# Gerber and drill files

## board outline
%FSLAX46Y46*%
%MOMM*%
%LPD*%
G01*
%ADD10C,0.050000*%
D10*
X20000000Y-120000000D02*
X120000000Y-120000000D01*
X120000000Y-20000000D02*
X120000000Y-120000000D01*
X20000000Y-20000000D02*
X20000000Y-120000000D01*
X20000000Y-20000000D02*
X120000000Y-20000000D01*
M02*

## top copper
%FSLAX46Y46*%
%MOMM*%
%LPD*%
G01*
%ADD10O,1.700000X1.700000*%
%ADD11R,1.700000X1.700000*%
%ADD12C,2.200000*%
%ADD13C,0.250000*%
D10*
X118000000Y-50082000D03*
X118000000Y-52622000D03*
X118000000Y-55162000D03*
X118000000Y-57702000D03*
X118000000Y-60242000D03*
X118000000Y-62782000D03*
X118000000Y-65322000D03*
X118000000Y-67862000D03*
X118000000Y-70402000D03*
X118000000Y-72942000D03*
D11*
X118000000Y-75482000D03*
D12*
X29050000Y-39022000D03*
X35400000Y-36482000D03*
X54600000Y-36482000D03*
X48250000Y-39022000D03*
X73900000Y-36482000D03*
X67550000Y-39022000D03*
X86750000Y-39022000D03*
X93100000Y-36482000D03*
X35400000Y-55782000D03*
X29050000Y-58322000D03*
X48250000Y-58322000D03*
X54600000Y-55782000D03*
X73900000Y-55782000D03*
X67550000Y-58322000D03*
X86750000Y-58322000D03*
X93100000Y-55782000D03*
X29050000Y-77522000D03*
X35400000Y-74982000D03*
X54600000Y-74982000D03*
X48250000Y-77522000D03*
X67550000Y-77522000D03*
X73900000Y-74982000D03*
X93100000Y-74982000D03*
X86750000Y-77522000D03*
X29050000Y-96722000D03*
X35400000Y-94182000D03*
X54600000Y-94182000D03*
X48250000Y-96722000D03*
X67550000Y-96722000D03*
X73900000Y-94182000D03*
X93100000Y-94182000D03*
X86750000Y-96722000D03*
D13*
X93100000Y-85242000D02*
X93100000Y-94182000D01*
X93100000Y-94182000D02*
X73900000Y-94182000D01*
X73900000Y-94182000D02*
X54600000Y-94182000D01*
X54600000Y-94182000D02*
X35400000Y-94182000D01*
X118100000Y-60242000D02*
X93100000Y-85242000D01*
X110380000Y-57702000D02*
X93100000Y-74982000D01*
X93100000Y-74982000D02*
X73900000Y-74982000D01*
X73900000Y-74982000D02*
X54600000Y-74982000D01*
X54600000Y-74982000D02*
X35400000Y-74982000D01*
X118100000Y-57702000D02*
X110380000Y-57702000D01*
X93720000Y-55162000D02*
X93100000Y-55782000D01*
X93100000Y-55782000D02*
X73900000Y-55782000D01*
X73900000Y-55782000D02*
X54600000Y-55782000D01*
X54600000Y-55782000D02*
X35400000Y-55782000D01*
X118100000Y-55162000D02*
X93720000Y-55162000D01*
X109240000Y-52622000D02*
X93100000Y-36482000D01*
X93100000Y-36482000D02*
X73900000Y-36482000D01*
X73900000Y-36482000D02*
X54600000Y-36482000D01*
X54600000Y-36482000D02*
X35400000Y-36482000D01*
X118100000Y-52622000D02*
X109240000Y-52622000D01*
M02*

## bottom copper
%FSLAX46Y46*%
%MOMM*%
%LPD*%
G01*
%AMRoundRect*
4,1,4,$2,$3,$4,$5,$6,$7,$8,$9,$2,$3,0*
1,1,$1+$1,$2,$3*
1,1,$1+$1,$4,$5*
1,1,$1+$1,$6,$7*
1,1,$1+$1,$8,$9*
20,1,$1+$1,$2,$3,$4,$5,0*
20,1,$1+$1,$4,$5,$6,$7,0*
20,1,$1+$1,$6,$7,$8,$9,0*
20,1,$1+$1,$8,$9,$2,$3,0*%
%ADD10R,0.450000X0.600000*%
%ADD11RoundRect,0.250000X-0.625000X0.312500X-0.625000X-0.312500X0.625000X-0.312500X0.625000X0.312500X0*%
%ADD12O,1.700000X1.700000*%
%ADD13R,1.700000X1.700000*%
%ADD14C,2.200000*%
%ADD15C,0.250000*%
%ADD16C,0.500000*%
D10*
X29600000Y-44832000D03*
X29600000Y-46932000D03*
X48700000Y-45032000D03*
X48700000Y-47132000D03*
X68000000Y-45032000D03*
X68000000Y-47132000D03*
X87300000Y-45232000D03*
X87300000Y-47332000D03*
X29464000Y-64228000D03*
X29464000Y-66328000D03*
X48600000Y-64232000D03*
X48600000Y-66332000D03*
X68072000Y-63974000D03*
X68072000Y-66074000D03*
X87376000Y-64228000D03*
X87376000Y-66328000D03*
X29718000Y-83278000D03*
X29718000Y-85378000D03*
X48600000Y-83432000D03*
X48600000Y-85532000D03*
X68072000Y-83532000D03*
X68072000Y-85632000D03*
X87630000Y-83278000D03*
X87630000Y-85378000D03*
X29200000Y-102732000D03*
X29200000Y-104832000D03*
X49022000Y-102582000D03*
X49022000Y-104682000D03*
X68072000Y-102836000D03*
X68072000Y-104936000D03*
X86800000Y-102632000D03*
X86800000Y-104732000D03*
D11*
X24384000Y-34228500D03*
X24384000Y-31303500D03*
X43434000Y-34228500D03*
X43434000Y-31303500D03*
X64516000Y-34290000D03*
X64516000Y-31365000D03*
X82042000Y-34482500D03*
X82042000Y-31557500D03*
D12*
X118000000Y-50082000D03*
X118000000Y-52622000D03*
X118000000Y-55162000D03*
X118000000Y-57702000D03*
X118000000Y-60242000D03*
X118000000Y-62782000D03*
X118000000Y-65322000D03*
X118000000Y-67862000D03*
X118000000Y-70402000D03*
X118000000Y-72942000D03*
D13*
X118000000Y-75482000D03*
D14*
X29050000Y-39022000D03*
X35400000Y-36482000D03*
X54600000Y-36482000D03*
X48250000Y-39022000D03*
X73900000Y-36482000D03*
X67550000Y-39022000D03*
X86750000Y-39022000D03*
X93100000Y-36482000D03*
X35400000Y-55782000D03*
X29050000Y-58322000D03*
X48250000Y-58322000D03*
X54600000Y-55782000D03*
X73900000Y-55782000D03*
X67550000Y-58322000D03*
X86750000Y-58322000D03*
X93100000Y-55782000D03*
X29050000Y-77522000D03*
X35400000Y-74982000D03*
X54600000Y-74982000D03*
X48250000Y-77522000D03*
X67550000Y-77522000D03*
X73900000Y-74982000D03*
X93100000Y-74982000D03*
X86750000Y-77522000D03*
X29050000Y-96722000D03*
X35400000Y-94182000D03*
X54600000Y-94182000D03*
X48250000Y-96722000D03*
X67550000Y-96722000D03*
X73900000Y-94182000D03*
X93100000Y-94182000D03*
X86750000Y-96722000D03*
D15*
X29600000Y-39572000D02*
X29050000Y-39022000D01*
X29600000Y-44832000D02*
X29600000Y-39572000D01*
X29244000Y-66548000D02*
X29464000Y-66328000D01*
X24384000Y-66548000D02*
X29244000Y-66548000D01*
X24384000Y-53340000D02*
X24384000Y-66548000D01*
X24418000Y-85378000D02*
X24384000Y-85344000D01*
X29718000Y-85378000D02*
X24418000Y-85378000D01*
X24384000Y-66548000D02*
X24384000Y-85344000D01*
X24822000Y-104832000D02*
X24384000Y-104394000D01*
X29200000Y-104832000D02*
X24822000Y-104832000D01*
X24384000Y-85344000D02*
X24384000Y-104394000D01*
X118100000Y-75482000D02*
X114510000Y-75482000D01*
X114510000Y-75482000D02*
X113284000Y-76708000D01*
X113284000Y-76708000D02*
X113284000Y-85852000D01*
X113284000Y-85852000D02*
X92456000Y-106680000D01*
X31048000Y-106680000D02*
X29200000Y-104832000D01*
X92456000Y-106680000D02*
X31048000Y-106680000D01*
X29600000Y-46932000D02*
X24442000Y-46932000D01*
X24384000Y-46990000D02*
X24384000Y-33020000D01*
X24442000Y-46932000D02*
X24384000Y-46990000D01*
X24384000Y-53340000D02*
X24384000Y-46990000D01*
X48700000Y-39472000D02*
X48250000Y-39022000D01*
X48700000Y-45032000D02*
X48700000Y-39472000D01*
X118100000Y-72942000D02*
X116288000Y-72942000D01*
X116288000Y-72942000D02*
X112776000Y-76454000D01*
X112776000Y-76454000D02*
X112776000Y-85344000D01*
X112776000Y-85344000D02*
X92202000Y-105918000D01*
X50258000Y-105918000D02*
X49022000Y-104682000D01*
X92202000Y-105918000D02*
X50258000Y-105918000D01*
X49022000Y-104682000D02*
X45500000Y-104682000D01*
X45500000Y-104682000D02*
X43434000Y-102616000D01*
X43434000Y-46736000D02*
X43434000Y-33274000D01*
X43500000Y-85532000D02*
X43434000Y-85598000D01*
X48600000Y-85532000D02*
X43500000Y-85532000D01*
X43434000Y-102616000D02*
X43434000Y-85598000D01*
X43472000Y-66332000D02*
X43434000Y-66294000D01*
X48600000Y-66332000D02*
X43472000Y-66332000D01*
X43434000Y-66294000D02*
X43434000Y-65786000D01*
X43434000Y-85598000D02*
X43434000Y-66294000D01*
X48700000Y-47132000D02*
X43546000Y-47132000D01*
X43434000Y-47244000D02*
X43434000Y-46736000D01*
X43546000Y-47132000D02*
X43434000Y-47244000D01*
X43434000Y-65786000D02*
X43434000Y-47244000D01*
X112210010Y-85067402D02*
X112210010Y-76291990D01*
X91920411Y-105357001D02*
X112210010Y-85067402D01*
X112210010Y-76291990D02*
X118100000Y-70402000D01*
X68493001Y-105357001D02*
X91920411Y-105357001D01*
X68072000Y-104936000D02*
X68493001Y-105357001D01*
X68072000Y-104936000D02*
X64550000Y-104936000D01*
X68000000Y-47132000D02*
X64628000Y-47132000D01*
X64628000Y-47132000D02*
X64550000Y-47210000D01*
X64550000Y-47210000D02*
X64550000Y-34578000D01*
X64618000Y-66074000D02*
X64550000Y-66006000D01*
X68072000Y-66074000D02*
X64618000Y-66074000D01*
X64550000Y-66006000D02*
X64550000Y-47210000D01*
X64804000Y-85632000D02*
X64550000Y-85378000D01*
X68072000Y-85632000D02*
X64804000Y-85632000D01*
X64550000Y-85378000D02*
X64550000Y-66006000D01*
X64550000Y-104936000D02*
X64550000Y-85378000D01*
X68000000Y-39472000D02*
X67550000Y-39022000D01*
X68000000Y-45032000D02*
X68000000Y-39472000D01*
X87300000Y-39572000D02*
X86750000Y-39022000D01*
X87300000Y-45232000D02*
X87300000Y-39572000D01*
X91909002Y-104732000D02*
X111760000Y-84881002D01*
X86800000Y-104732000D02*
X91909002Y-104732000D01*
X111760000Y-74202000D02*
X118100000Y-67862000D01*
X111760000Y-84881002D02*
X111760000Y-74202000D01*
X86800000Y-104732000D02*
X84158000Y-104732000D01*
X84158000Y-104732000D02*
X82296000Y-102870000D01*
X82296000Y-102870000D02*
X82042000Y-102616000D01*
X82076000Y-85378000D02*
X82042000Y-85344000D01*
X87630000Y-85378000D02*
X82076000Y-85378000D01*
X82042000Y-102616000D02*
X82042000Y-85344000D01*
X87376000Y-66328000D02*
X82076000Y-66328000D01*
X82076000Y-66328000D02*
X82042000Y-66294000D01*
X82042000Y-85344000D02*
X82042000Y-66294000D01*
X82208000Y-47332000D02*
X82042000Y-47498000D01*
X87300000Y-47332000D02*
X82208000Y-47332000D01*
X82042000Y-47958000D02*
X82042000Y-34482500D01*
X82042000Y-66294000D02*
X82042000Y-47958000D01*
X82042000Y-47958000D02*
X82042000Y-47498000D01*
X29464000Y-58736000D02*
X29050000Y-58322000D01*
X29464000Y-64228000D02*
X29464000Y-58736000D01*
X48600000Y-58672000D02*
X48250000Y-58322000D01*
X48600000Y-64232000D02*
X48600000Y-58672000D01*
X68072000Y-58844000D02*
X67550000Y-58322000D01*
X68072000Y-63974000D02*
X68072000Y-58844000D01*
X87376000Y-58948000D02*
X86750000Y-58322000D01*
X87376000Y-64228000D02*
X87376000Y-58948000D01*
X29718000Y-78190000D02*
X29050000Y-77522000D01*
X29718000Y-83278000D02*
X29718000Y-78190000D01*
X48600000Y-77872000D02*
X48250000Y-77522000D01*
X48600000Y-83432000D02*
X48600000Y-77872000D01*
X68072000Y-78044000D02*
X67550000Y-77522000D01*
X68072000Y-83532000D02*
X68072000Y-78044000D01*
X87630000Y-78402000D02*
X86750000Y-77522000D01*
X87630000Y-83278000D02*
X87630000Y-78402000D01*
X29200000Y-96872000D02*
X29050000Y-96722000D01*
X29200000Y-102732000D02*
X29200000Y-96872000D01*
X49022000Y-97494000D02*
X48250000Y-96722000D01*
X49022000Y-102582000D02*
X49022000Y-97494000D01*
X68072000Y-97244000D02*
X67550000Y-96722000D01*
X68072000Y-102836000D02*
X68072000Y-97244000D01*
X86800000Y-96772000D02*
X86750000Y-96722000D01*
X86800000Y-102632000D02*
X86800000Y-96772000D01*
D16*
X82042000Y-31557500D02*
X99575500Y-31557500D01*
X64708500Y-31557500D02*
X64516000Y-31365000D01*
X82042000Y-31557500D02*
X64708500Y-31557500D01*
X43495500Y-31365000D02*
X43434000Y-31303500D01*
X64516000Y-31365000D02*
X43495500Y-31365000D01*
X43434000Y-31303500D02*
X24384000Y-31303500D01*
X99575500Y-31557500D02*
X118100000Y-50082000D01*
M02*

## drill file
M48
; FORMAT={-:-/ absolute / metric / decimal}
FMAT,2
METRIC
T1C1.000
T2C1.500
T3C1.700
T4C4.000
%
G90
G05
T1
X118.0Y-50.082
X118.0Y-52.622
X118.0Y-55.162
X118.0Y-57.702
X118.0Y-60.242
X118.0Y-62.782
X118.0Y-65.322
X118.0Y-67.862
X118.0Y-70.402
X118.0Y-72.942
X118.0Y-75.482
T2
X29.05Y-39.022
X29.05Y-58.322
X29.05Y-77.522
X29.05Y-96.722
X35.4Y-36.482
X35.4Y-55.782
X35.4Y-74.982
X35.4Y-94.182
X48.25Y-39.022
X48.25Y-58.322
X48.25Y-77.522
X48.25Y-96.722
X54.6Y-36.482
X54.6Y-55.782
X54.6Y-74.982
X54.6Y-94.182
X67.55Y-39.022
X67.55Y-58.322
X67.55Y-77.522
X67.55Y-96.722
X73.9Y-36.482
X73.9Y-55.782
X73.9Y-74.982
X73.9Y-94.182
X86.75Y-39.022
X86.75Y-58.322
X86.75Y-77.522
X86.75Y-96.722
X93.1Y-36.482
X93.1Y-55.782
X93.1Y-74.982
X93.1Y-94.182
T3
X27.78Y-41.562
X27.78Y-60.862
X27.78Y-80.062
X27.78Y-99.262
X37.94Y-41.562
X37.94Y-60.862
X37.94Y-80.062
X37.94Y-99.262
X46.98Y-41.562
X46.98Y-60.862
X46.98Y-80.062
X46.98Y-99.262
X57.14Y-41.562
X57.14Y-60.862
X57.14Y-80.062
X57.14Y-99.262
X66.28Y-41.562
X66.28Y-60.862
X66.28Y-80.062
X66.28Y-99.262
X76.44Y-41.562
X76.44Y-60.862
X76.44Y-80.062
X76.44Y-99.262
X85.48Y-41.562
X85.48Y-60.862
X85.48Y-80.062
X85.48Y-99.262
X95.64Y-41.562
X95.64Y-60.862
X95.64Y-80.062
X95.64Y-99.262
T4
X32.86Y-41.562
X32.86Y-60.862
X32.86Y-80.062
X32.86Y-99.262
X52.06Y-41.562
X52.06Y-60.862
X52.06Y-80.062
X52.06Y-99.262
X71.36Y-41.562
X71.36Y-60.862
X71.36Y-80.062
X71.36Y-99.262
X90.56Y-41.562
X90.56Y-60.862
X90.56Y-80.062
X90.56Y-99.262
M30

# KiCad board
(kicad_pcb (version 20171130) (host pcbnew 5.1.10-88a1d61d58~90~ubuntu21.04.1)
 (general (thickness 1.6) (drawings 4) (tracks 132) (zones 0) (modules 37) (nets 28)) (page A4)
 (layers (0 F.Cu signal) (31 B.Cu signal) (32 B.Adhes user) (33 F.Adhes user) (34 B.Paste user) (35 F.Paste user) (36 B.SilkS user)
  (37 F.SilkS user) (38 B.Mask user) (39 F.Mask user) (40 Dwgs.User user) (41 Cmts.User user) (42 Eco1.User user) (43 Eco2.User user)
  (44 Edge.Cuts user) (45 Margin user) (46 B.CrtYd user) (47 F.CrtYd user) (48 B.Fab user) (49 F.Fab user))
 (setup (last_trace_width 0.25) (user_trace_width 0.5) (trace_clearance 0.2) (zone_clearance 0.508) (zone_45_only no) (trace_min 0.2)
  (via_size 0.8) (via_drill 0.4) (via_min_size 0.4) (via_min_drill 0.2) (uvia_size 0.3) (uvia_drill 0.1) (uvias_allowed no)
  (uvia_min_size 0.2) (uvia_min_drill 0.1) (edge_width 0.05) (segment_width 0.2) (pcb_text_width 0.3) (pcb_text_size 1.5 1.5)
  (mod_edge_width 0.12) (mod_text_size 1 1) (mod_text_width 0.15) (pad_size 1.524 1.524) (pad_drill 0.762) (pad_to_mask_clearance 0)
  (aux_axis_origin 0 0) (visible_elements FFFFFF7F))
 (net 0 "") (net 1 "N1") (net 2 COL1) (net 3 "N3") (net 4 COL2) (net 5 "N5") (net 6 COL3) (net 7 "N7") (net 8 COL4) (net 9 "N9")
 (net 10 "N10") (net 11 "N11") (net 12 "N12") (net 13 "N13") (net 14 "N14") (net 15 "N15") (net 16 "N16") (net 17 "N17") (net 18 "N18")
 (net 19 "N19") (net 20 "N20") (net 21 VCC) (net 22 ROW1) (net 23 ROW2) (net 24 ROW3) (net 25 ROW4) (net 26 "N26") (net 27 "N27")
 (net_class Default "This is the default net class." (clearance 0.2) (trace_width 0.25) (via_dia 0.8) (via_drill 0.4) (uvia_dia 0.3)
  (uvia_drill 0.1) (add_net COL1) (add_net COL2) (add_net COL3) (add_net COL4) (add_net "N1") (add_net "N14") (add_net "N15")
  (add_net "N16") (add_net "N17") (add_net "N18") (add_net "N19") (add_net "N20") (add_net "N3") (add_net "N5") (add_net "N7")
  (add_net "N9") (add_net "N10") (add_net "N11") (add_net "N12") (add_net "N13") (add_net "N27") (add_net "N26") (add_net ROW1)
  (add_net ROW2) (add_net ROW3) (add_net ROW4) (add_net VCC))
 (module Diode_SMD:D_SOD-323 (layer B.Cu) (at 29.6 45.882 90)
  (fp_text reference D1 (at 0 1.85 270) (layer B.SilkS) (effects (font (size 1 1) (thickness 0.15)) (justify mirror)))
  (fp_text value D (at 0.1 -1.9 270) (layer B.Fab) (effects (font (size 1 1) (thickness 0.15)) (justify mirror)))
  (pad 2 smd rect (at 1.05 0 90) (size 0.6 0.45) (layers B.Cu B.Paste B.Mask) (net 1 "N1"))
  (pad 1 smd rect (at -1.05 0 90) (size 0.6 0.45) (layers B.Cu B.Paste B.Mask) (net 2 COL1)))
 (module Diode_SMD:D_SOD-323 (layer B.Cu) (at 48.7 46.082 90)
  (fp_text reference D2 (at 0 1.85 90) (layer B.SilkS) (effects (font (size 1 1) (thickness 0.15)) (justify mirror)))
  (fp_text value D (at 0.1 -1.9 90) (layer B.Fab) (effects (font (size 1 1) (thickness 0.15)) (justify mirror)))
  (pad 2 smd rect (at 1.05 0 90) (size 0.6 0.45) (layers B.Cu B.Paste B.Mask) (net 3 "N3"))
  (pad 1 smd rect (at -1.05 0 90) (size 0.6 0.45) (layers B.Cu B.Paste B.Mask) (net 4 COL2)))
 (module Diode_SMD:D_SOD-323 (layer B.Cu) (at 68 46.082 90)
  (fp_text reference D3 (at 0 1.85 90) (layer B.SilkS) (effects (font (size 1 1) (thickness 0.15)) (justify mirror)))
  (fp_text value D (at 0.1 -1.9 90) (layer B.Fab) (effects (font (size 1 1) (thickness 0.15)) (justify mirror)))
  (pad 2 smd rect (at 1.05 0 90) (size 0.6 0.45) (layers B.Cu B.Paste B.Mask) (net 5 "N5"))
  (pad 1 smd rect (at -1.05 0 90) (size 0.6 0.45) (layers B.Cu B.Paste B.Mask) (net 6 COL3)))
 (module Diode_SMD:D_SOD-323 (layer B.Cu) (at 87.3 46.282 90)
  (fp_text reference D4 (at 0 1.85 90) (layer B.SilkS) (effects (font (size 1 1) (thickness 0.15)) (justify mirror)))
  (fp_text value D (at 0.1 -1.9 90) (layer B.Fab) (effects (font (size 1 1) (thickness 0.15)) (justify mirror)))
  (pad 2 smd rect (at 1.05 0 90) (size 0.6 0.45) (layers B.Cu B.Paste B.Mask) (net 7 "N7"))
  (pad 1 smd rect (at -1.05 0 90) (size 0.6 0.45) (layers B.Cu B.Paste B.Mask) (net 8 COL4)))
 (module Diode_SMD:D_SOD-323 (layer B.Cu) (at 29.464 65.278 90)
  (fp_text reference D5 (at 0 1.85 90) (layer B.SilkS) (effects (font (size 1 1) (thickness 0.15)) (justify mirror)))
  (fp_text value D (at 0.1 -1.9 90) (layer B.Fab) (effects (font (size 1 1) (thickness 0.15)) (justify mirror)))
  (pad 2 smd rect (at 1.05 0 90) (size 0.6 0.45) (layers B.Cu B.Paste B.Mask) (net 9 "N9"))
  (pad 1 smd rect (at -1.05 0 90) (size 0.6 0.45) (layers B.Cu B.Paste B.Mask) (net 2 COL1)))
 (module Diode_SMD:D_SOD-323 (layer B.Cu) (at 48.6 65.282 90)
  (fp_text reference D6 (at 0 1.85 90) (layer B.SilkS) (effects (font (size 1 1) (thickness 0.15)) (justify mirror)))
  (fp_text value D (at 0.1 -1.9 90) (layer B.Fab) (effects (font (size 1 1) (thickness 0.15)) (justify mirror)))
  (pad 2 smd rect (at 1.05 0 90) (size 0.6 0.45) (layers B.Cu B.Paste B.Mask) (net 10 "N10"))
  (pad 1 smd rect (at -1.05 0 90) (size 0.6 0.45) (layers B.Cu B.Paste B.Mask) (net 4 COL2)))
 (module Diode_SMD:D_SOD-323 (layer B.Cu) (at 68.072 65.024 90)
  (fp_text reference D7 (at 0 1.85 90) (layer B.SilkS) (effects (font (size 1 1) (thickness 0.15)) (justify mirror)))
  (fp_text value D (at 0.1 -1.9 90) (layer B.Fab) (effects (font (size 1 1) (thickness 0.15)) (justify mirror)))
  (pad 2 smd rect (at 1.05 0 90) (size 0.6 0.45) (layers B.Cu B.Paste B.Mask) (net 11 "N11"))
  (pad 1 smd rect (at -1.05 0 90) (size 0.6 0.45) (layers B.Cu B.Paste B.Mask) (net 6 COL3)))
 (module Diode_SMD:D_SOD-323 (layer B.Cu) (at 87.376 65.278 90)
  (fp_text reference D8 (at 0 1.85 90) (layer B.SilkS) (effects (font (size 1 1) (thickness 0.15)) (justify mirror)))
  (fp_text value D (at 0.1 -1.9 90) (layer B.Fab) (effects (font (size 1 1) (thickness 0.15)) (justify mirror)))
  (pad 2 smd rect (at 1.05 0 90) (size 0.6 0.45) (layers B.Cu B.Paste B.Mask) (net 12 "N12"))
  (pad 1 smd rect (at -1.05 0 90) (size 0.6 0.45) (layers B.Cu B.Paste B.Mask) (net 8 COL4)))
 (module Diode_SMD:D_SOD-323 (layer B.Cu) (at 29.718 84.328 90)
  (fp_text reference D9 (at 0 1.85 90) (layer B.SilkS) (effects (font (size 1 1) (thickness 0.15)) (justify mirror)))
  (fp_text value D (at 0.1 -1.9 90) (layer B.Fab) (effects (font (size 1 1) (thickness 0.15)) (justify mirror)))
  (pad 2 smd rect (at 1.05 0 90) (size 0.6 0.45) (layers B.Cu B.Paste B.Mask) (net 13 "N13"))
  (pad 1 smd rect (at -1.05 0 90) (size 0.6 0.45) (layers B.Cu B.Paste B.Mask) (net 2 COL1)))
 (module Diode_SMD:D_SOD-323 (layer B.Cu) (at 48.6 84.482 90)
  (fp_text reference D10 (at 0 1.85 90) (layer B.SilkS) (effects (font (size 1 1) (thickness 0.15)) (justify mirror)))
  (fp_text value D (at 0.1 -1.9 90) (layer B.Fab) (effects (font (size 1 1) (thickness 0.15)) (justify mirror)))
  (pad 2 smd rect (at 1.05 0 90) (size 0.6 0.45) (layers B.Cu B.Paste B.Mask) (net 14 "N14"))
  (pad 1 smd rect (at -1.05 0 90) (size 0.6 0.45) (layers B.Cu B.Paste B.Mask) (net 4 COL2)))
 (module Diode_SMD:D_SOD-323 (layer B.Cu) (at 68.072 84.582 90)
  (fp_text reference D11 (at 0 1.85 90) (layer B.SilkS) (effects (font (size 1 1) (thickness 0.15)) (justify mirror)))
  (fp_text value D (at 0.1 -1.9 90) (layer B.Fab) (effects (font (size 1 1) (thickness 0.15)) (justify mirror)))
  (pad 2 smd rect (at 1.05 0 90) (size 0.6 0.45) (layers B.Cu B.Paste B.Mask) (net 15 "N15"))
  (pad 1 smd rect (at -1.05 0 90) (size 0.6 0.45) (layers B.Cu B.Paste B.Mask) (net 6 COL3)))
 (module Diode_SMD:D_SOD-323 (layer B.Cu) (at 87.63 84.328 90)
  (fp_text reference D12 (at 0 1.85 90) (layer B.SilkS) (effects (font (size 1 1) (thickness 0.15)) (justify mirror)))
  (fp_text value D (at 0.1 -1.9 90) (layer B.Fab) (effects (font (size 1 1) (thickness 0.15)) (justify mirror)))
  (pad 2 smd rect (at 1.05 0 90) (size 0.6 0.45) (layers B.Cu B.Paste B.Mask) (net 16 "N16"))
  (pad 1 smd rect (at -1.05 0 90) (size 0.6 0.45) (layers B.Cu B.Paste B.Mask) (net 8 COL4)))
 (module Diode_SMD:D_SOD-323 (layer B.Cu) (at 29.2 103.782 90)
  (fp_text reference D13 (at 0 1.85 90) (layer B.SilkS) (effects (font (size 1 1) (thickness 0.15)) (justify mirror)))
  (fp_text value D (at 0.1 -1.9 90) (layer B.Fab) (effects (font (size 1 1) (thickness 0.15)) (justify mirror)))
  (pad 2 smd rect (at 1.05 0 90) (size 0.6 0.45) (layers B.Cu B.Paste B.Mask) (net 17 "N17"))
  (pad 1 smd rect (at -1.05 0 90) (size 0.6 0.45) (layers B.Cu B.Paste B.Mask) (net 2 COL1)))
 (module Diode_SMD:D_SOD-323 (layer B.Cu) (at 49.022 103.632 90)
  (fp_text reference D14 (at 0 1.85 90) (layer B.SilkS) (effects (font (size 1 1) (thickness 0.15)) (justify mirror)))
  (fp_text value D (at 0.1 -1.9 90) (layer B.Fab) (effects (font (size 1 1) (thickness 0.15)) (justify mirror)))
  (pad 2 smd rect (at 1.05 0 90) (size 0.6 0.45) (layers B.Cu B.Paste B.Mask) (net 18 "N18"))
  (pad 1 smd rect (at -1.05 0 90) (size 0.6 0.45) (layers B.Cu B.Paste B.Mask) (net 4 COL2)))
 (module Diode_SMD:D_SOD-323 (layer B.Cu) (at 68.072 103.886 90)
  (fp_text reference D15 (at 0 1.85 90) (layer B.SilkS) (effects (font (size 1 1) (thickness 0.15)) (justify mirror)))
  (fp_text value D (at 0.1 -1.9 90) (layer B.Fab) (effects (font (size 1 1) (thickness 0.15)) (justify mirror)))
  (pad 2 smd rect (at 1.05 0 90) (size 0.6 0.45) (layers B.Cu B.Paste B.Mask) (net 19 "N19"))
  (pad 1 smd rect (at -1.05 0 90) (size 0.6 0.45) (layers B.Cu B.Paste B.Mask) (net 6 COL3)))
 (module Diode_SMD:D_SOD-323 (layer B.Cu) (at 86.8 103.682 90)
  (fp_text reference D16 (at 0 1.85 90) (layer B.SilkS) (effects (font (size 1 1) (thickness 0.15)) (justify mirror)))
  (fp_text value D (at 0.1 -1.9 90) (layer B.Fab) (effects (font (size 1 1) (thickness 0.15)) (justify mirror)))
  (pad 2 smd rect (at 1.05 0 90) (size 0.6 0.45) (layers B.Cu B.Paste B.Mask) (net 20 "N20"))
  (pad 1 smd rect (at -1.05 0 90) (size 0.6 0.45) (layers B.Cu B.Paste B.Mask) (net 8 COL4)))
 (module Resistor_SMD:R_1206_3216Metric (layer B.Cu) (at 24.384 32.766 270)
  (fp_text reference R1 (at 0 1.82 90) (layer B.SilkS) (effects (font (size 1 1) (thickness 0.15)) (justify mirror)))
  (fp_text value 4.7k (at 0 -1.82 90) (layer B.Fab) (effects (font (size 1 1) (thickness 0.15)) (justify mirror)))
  (pad 2 smd roundrect (at 1.4625 0 270) (size 1.125 1.75) (layers B.Cu B.Paste B.Mask) (roundrect_rratio 0.222222) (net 2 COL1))
  (pad 1 smd roundrect (at -1.4625 0 270) (size 1.125 1.75) (layers B.Cu B.Paste B.Mask) (roundrect_rratio 0.222222) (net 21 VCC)))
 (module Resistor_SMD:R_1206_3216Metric (layer B.Cu) (at 43.434 32.766 270)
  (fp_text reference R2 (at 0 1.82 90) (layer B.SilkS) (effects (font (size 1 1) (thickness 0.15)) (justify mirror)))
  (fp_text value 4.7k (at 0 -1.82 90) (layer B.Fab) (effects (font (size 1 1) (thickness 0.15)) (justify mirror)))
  (pad 2 smd roundrect (at 1.4625 0 270) (size 1.125 1.75) (layers B.Cu B.Paste B.Mask) (roundrect_rratio 0.222222) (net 4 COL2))
  (pad 1 smd roundrect (at -1.4625 0 270) (size 1.125 1.75) (layers B.Cu B.Paste B.Mask) (roundrect_rratio 0.222222) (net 21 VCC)))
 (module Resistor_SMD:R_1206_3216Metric (layer B.Cu) (at 64.516 32.8275 270)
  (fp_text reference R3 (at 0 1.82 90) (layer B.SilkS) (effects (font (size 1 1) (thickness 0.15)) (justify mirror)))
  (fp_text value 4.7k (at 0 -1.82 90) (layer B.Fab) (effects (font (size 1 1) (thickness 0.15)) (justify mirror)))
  (pad 2 smd roundrect (at 1.4625 0 270) (size 1.125 1.75) (layers B.Cu B.Paste B.Mask) (roundrect_rratio 0.222222) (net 6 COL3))
  (pad 1 smd roundrect (at -1.4625 0 270) (size 1.125 1.75) (layers B.Cu B.Paste B.Mask) (roundrect_rratio 0.222222) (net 21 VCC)))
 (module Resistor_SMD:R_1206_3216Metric (layer B.Cu) (at 82.042 33.02 270)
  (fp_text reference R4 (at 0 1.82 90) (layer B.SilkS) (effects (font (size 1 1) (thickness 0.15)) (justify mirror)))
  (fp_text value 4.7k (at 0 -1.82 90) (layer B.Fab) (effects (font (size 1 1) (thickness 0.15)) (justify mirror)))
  (pad 2 smd roundrect (at 1.4625 0 270) (size 1.125 1.75) (layers B.Cu B.Paste B.Mask) (roundrect_rratio 0.222222) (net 8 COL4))
  (pad 1 smd roundrect (at -1.4625 0 270) (size 1.125 1.75) (layers B.Cu B.Paste B.Mask) (roundrect_rratio 0.222222) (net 21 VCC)))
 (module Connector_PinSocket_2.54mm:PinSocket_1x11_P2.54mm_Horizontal (layer F.Cu) (at 118 75.482 180)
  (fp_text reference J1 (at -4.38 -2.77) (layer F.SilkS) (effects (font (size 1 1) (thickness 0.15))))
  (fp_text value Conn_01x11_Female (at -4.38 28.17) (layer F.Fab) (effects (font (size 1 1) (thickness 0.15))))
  (pad 11 thru_hole oval (at 0 25.4 180) (size 1.7 1.7) (drill 1) (layers *.Cu *.Mask) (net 21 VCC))
  (pad 10 thru_hole oval (at 0 22.86 180) (size 1.7 1.7) (drill 1) (layers *.Cu *.Mask) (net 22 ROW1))
  (pad 9 thru_hole oval (at 0 20.32 180) (size 1.7 1.7) (drill 1) (layers *.Cu *.Mask) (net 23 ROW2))
  (pad 8 thru_hole oval (at 0 17.78 180) (size 1.7 1.7) (drill 1) (layers *.Cu *.Mask) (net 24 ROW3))
  (pad 7 thru_hole oval (at 0 15.24 180) (size 1.7 1.7) (drill 1) (layers *.Cu *.Mask) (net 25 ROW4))
  (pad 6 thru_hole oval (at 0 12.7 180) (size 1.7 1.7) (drill 1) (layers *.Cu *.Mask) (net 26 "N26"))
  (pad 5 thru_hole oval (at 0 10.16 180) (size 1.7 1.7) (drill 1) (layers *.Cu *.Mask) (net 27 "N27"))
  (pad 4 thru_hole oval (at 0 7.62 180) (size 1.7 1.7) (drill 1) (layers *.Cu *.Mask) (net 8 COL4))
  (pad 3 thru_hole oval (at 0 5.08 180) (size 1.7 1.7) (drill 1) (layers *.Cu *.Mask) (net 6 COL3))
  (pad 2 thru_hole oval (at 0 2.54 180) (size 1.7 1.7) (drill 1) (layers *.Cu *.Mask) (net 4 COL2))
  (pad 1 thru_hole rect (at 0 0 180) (size 1.7 1.7) (drill 1) (layers *.Cu *.Mask) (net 2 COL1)))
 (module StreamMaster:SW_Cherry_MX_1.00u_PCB (layer F.Cu) (at 35.4 36.482)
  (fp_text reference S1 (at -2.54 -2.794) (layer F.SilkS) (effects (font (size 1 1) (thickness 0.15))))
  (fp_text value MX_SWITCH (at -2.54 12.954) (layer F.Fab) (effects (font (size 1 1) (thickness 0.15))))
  (pad "" np_thru_hole circle (at 2.54 5.08) (size 1.7 1.7) (drill 1.7) (layers *.Cu *.Mask))
  (pad "" np_thru_hole circle (at -7.62 5.08) (size 1.7 1.7) (drill 1.7) (layers *.Cu *.Mask))
  (pad "" np_thru_hole circle (at -2.54 5.08) (size 4 4) (drill 4) (layers *.Cu *.Mask))
  (pad 2 thru_hole circle (at -6.35 2.54) (size 2.2 2.2) (drill 1.5) (layers *.Cu *.Mask) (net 1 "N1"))
  (pad 1 thru_hole circle (at 0 0) (size 2.2 2.2) (drill 1.5) (layers *.Cu *.Mask) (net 22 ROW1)))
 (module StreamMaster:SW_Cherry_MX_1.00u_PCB (layer F.Cu) (at 54.6 36.482)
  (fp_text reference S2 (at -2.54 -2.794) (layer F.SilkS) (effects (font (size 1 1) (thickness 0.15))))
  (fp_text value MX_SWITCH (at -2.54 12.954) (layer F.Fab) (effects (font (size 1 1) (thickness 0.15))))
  (pad 1 thru_hole circle (at 0 0) (size 2.2 2.2) (drill 1.5) (layers *.Cu *.Mask) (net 22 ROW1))
  (pad 2 thru_hole circle (at -6.35 2.54) (size 2.2 2.2) (drill 1.5) (layers *.Cu *.Mask) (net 3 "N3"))
  (pad "" np_thru_hole circle (at -2.54 5.08) (size 4 4) (drill 4) (layers *.Cu *.Mask))
  (pad "" np_thru_hole circle (at -7.62 5.08) (size 1.7 1.7) (drill 1.7) (layers *.Cu *.Mask))
  (pad "" np_thru_hole circle (at 2.54 5.08) (size 1.7 1.7) (drill 1.7) (layers *.Cu *.Mask)))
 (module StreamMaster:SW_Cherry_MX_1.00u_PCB (layer F.Cu) (at 73.9 36.482)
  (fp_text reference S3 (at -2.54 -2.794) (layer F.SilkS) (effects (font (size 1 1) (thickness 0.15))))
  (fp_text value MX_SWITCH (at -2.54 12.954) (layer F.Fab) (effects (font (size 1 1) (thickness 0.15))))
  (pad 1 thru_hole circle (at 0 0) (size 2.2 2.2) (drill 1.5) (layers *.Cu *.Mask) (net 22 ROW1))
  (pad 2 thru_hole circle (at -6.35 2.54) (size 2.2 2.2) (drill 1.5) (layers *.Cu *.Mask) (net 5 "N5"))
  (pad "" np_thru_hole circle (at -2.54 5.08) (size 4 4) (drill 4) (layers *.Cu *.Mask))
  (pad "" np_thru_hole circle (at -7.62 5.08) (size 1.7 1.7) (drill 1.7) (layers *.Cu *.Mask))
  (pad "" np_thru_hole circle (at 2.54 5.08) (size 1.7 1.7) (drill 1.7) (layers *.Cu *.Mask)))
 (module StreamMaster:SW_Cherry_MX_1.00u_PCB (layer F.Cu) (at 93.1 36.482)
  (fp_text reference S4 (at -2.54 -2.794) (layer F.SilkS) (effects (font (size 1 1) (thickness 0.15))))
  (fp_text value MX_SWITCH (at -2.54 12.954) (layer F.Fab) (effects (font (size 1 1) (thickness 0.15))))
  (pad "" np_thru_hole circle (at 2.54 5.08) (size 1.7 1.7) (drill 1.7) (layers *.Cu *.Mask))
  (pad "" np_thru_hole circle (at -7.62 5.08) (size 1.7 1.7) (drill 1.7) (layers *.Cu *.Mask))
  (pad "" np_thru_hole circle (at -2.54 5.08) (size 4 4) (drill 4) (layers *.Cu *.Mask))
  (pad 2 thru_hole circle (at -6.35 2.54) (size 2.2 2.2) (drill 1.5) (layers *.Cu *.Mask) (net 7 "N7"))
  (pad 1 thru_hole circle (at 0 0) (size 2.2 2.2) (drill 1.5) (layers *.Cu *.Mask) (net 22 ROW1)))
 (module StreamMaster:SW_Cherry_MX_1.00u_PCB (layer F.Cu) (at 35.4 55.782)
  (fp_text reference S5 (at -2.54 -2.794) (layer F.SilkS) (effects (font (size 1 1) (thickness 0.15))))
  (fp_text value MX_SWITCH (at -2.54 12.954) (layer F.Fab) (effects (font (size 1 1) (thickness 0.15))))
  (pad 1 thru_hole circle (at 0 0) (size 2.2 2.2) (drill 1.5) (layers *.Cu *.Mask) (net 23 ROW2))
  (pad 2 thru_hole circle (at -6.35 2.54) (size 2.2 2.2) (drill 1.5) (layers *.Cu *.Mask) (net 9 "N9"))
  (pad "" np_thru_hole circle (at -2.54 5.08) (size 4 4) (drill 4) (layers *.Cu *.Mask))
  (pad "" np_thru_hole circle (at -7.62 5.08) (size 1.7 1.7) (drill 1.7) (layers *.Cu *.Mask))
  (pad "" np_thru_hole circle (at 2.54 5.08) (size 1.7 1.7) (drill 1.7) (layers *.Cu *.Mask)))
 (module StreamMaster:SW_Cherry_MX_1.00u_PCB (layer F.Cu) (at 54.6 55.782)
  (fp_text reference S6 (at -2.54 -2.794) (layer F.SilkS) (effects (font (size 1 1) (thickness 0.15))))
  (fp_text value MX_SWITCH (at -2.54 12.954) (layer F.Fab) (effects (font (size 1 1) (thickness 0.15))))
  (pad "" np_thru_hole circle (at 2.54 5.08) (size 1.7 1.7) (drill 1.7) (layers *.Cu *.Mask))
  (pad "" np_thru_hole circle (at -7.62 5.08) (size 1.7 1.7) (drill 1.7) (layers *.Cu *.Mask))
  (pad "" np_thru_hole circle (at -2.54 5.08) (size 4 4) (drill 4) (layers *.Cu *.Mask))
  (pad 2 thru_hole circle (at -6.35 2.54) (size 2.2 2.2) (drill 1.5) (layers *.Cu *.Mask) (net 10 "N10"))
  (pad 1 thru_hole circle (at 0 0) (size 2.2 2.2) (drill 1.5) (layers *.Cu *.Mask) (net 23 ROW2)))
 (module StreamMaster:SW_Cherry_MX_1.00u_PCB (layer F.Cu) (at 73.9 55.782)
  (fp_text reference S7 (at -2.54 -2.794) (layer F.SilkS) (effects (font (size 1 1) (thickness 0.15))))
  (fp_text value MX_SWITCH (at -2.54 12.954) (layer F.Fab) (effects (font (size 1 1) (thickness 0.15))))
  (pad 1 thru_hole circle (at 0 0) (size 2.2 2.2) (drill 1.5) (layers *.Cu *.Mask) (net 23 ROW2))
  (pad 2 thru_hole circle (at -6.35 2.54) (size 2.2 2.2) (drill 1.5) (layers *.Cu *.Mask) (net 11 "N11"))
  (pad "" np_thru_hole circle (at -2.54 5.08) (size 4 4) (drill 4) (layers *.Cu *.Mask))
  (pad "" np_thru_hole circle (at -7.62 5.08) (size 1.7 1.7) (drill 1.7) (layers *.Cu *.Mask))
  (pad "" np_thru_hole circle (at 2.54 5.08) (size 1.7 1.7) (drill 1.7) (layers *.Cu *.Mask)))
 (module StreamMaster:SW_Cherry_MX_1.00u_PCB (layer F.Cu) (at 93.1 55.782)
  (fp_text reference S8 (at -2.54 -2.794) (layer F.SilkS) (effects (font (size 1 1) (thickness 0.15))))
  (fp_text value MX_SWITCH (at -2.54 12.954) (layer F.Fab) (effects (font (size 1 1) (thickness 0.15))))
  (pad "" np_thru_hole circle (at 2.54 5.08) (size 1.7 1.7) (drill 1.7) (layers *.Cu *.Mask))
  (pad "" np_thru_hole circle (at -7.62 5.08) (size 1.7 1.7) (drill 1.7) (layers *.Cu *.Mask))
  (pad "" np_thru_hole circle (at -2.54 5.08) (size 4 4) (drill 4) (layers *.Cu *.Mask))
  (pad 2 thru_hole circle (at -6.35 2.54) (size 2.2 2.2) (drill 1.5) (layers *.Cu *.Mask) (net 12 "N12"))
  (pad 1 thru_hole circle (at 0 0) (size 2.2 2.2) (drill 1.5) (layers *.Cu *.Mask) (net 23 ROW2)))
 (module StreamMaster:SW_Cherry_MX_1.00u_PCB (layer F.Cu) (at 35.4 74.982)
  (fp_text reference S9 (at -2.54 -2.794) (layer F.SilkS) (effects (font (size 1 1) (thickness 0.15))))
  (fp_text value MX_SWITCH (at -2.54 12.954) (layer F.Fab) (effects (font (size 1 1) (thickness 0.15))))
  (pad "" np_thru_hole circle (at 2.54 5.08) (size 1.7 1.7) (drill 1.7) (layers *.Cu *.Mask))
  (pad "" np_thru_hole circle (at -7.62 5.08) (size 1.7 1.7) (drill 1.7) (layers *.Cu *.Mask))
  (pad "" np_thru_hole circle (at -2.54 5.08) (size 4 4) (drill 4) (layers *.Cu *.Mask))
  (pad 2 thru_hole circle (at -6.35 2.54) (size 2.2 2.2) (drill 1.5) (layers *.Cu *.Mask) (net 13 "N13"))
  (pad 1 thru_hole circle (at 0 0) (size 2.2 2.2) (drill 1.5) (layers *.Cu *.Mask) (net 24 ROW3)))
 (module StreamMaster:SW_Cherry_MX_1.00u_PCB (layer F.Cu) (at 54.6 74.982)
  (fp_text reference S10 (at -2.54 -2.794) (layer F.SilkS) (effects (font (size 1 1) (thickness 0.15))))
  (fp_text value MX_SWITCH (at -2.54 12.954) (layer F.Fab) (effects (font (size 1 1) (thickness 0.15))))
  (pad 1 thru_hole circle (at 0 0) (size 2.2 2.2) (drill 1.5) (layers *.Cu *.Mask) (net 24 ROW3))
  (pad 2 thru_hole circle (at -6.35 2.54) (size 2.2 2.2) (drill 1.5) (layers *.Cu *.Mask) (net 14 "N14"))
  (pad "" np_thru_hole circle (at -2.54 5.08) (size 4 4) (drill 4) (layers *.Cu *.Mask))
  (pad "" np_thru_hole circle (at -7.62 5.08) (size 1.7 1.7) (drill 1.7) (layers *.Cu *.Mask))
  (pad "" np_thru_hole circle (at 2.54 5.08) (size 1.7 1.7) (drill 1.7) (layers *.Cu *.Mask)))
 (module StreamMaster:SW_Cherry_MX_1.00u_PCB (layer F.Cu) (at 73.9 74.982)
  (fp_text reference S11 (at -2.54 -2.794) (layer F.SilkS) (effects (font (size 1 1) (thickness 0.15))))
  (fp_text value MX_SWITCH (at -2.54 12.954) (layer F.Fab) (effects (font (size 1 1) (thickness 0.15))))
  (pad "" np_thru_hole circle (at 2.54 5.08) (size 1.7 1.7) (drill 1.7) (layers *.Cu *.Mask))
  (pad "" np_thru_hole circle (at -7.62 5.08) (size 1.7 1.7) (drill 1.7) (layers *.Cu *.Mask))
  (pad "" np_thru_hole circle (at -2.54 5.08) (size 4 4) (drill 4) (layers *.Cu *.Mask))
  (pad 2 thru_hole circle (at -6.35 2.54) (size 2.2 2.2) (drill 1.5) (layers *.Cu *.Mask) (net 15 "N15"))
  (pad 1 thru_hole circle (at 0 0) (size 2.2 2.2) (drill 1.5) (layers *.Cu *.Mask) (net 24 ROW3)))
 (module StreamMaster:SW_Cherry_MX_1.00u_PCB (layer F.Cu) (at 93.1 74.982)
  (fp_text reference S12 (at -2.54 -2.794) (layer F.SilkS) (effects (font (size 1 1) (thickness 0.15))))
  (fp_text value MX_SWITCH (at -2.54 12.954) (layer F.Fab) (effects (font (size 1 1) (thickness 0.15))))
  (pad 1 thru_hole circle (at 0 0) (size 2.2 2.2) (drill 1.5) (layers *.Cu *.Mask) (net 24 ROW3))
  (pad 2 thru_hole circle (at -6.35 2.54) (size 2.2 2.2) (drill 1.5) (layers *.Cu *.Mask) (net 16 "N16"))
  (pad "" np_thru_hole circle (at -2.54 5.08) (size 4 4) (drill 4) (layers *.Cu *.Mask))
  (pad "" np_thru_hole circle (at -7.62 5.08) (size 1.7 1.7) (drill 1.7) (layers *.Cu *.Mask))
  (pad "" np_thru_hole circle (at 2.54 5.08) (size 1.7 1.7) (drill 1.7) (layers *.Cu *.Mask)))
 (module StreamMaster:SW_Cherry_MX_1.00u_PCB (layer F.Cu) (at 35.4 94.182)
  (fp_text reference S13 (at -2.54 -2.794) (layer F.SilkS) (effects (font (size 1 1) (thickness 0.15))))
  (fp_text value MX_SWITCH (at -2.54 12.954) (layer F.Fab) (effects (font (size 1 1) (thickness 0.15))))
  (pad "" np_thru_hole circle (at 2.54 5.08) (size 1.7 1.7) (drill 1.7) (layers *.Cu *.Mask))
  (pad "" np_thru_hole circle (at -7.62 5.08) (size 1.7 1.7) (drill 1.7) (layers *.Cu *.Mask))
  (pad "" np_thru_hole circle (at -2.54 5.08) (size 4 4) (drill 4) (layers *.Cu *.Mask))
  (pad 2 thru_hole circle (at -6.35 2.54) (size 2.2 2.2) (drill 1.5) (layers *.Cu *.Mask) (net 17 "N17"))
  (pad 1 thru_hole circle (at 0 0) (size 2.2 2.2) (drill 1.5) (layers *.Cu *.Mask) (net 25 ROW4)))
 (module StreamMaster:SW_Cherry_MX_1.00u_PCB (layer F.Cu) (at 54.6 94.182)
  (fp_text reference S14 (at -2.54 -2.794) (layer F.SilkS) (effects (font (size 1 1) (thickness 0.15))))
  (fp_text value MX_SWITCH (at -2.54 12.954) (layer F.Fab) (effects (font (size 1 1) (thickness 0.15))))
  (pad 1 thru_hole circle (at 0 0) (size 2.2 2.2) (drill 1.5) (layers *.Cu *.Mask) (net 25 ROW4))
  (pad 2 thru_hole circle (at -6.35 2.54) (size 2.2 2.2) (drill 1.5) (layers *.Cu *.Mask) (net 18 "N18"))
  (pad "" np_thru_hole circle (at -2.54 5.08) (size 4 4) (drill 4) (layers *.Cu *.Mask))
  (pad "" np_thru_hole circle (at -7.62 5.08) (size 1.7 1.7) (drill 1.7) (layers *.Cu *.Mask))
  (pad "" np_thru_hole circle (at 2.54 5.08) (size 1.7 1.7) (drill 1.7) (layers *.Cu *.Mask)))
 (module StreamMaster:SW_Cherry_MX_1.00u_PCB (layer F.Cu) (at 73.9 94.182)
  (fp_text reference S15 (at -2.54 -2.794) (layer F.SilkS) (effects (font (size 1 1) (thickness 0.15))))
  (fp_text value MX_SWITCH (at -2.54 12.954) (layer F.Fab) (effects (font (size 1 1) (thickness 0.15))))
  (pad "" np_thru_hole circle (at 2.54 5.08) (size 1.7 1.7) (drill 1.7) (layers *.Cu *.Mask))
  (pad "" np_thru_hole circle (at -7.62 5.08) (size 1.7 1.7) (drill 1.7) (layers *.Cu *.Mask))
  (pad "" np_thru_hole circle (at -2.54 5.08) (size 4 4) (drill 4) (layers *.Cu *.Mask))
  (pad 2 thru_hole circle (at -6.35 2.54) (size 2.2 2.2) (drill 1.5) (layers *.Cu *.Mask) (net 19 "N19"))
  (pad 1 thru_hole circle (at 0 0) (size 2.2 2.2) (drill 1.5) (layers *.Cu *.Mask) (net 25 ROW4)))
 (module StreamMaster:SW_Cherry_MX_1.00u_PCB (layer F.Cu) (at 93.1 94.182)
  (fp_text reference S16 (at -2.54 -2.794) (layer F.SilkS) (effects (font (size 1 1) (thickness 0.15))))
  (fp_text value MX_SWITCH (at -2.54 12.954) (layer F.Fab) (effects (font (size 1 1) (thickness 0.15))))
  (pad 1 thru_hole circle (at 0 0) (size 2.2 2.2) (drill 1.5) (layers *.Cu *.Mask) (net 25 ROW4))
  (pad 2 thru_hole circle (at -6.35 2.54) (size 2.2 2.2) (drill 1.5) (layers *.Cu *.Mask) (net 20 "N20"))
  (pad "" np_thru_hole circle (at -2.54 5.08) (size 4 4) (drill 4) (layers *.Cu *.Mask))
  (pad "" np_thru_hole circle (at -7.62 5.08) (size 1.7 1.7) (drill 1.7) (layers *.Cu *.Mask))
  (pad "" np_thru_hole circle (at 2.54 5.08) (size 1.7 1.7) (drill 1.7) (layers *.Cu *.Mask)))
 (gr_line (start 20 120) (end 120 120) (layer Edge.Cuts) (width 0.05))
 (gr_line (start 120 20) (end 120 120) (layer Edge.Cuts) (width 0.05))
 (gr_line (start 20 20) (end 20 120) (layer Edge.Cuts) (width 0.05))
 (gr_line (start 20 20) (end 120 20) (layer Edge.Cuts) (width 0.05))
 (segment (start 29.6 39.572) (end 29.05 39.022) (width 0.25) (layer B.Cu) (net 1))
 (segment (start 29.6 44.832) (end 29.6 39.572) (width 0.25) (layer B.Cu) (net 1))
 (segment (start 29.244 66.548) (end 29.464 66.328) (width 0.25) (layer B.Cu) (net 2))
 (segment (start 24.384 66.548) (end 29.244 66.548) (width 0.25) (layer B.Cu) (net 2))
 (segment (start 24.384 53.34) (end 24.384 66.548) (width 0.25) (layer B.Cu) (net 2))
 (segment (start 24.418 85.378) (end 24.384 85.344) (width 0.25) (layer B.Cu) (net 2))
 (segment (start 29.718 85.378) (end 24.418 85.378) (width 0.25) (layer B.Cu) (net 2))
 (segment (start 24.384 66.548) (end 24.384 85.344) (width 0.25) (layer B.Cu) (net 2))
 (segment (start 24.822 104.832) (end 24.384 104.394) (width 0.25) (layer B.Cu) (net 2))
 (segment (start 29.2 104.832) (end 24.822 104.832) (width 0.25) (layer B.Cu) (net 2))
 (segment (start 24.384 85.344) (end 24.384 104.394) (width 0.25) (layer B.Cu) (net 2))
 (segment (start 118.1 75.482) (end 114.51 75.482) (width 0.25) (layer B.Cu) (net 2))
 (segment (start 114.51 75.482) (end 113.284 76.708) (width 0.25) (layer B.Cu) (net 2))
 (segment (start 113.284 76.708) (end 113.284 85.852) (width 0.25) (layer B.Cu) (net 2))
 (segment (start 113.284 85.852) (end 92.456 106.68) (width 0.25) (layer B.Cu) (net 2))
 (segment (start 31.048 106.68) (end 29.2 104.832) (width 0.25) (layer B.Cu) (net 2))
 (segment (start 92.456 106.68) (end 31.048 106.68) (width 0.25) (layer B.Cu) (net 2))
 (segment (start 29.6 46.932) (end 24.442 46.932) (width 0.25) (layer B.Cu) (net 2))
 (segment (start 24.384 46.99) (end 24.384 33.02) (width 0.25) (layer B.Cu) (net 2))
 (segment (start 24.442 46.932) (end 24.384 46.99) (width 0.25) (layer B.Cu) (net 2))
 (segment (start 24.384 53.34) (end 24.384 46.99) (width 0.25) (layer B.Cu) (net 2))
 (segment (start 48.7 39.472) (end 48.25 39.022) (width 0.25) (layer B.Cu) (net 3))
 (segment (start 48.7 45.032) (end 48.7 39.472) (width 0.25) (layer B.Cu) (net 3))
 (segment (start 118.1 72.942) (end 116.288 72.942) (width 0.25) (layer B.Cu) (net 4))
 (segment (start 116.288 72.942) (end 112.776 76.454) (width 0.25) (layer B.Cu) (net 4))
 (segment (start 112.776 76.454) (end 112.776 85.344) (width 0.25) (layer B.Cu) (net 4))
 (segment (start 112.776 85.344) (end 92.202 105.918) (width 0.25) (layer B.Cu) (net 4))
 (segment (start 50.258 105.918) (end 49.022 104.682) (width 0.25) (layer B.Cu) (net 4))
 (segment (start 92.202 105.918) (end 50.258 105.918) (width 0.25) (layer B.Cu) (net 4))
 (segment (start 49.022 104.682) (end 45.5 104.682) (width 0.25) (layer B.Cu) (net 4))
 (segment (start 45.5 104.682) (end 43.434 102.616) (width 0.25) (layer B.Cu) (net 4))
 (segment (start 43.434 46.736) (end 43.434 33.274) (width 0.25) (layer B.Cu) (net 4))
 (segment (start 43.5 85.532) (end 43.434 85.598) (width 0.25) (layer B.Cu) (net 4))
 (segment (start 48.6 85.532) (end 43.5 85.532) (width 0.25) (layer B.Cu) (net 4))
 (segment (start 43.434 102.616) (end 43.434 85.598) (width 0.25) (layer B.Cu) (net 4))
 (segment (start 43.472 66.332) (end 43.434 66.294) (width 0.25) (layer B.Cu) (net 4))
 (segment (start 48.6 66.332) (end 43.472 66.332) (width 0.25) (layer B.Cu) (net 4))
 (segment (start 43.434 66.294) (end 43.434 65.786) (width 0.25) (layer B.Cu) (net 4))
 (segment (start 43.434 85.598) (end 43.434 66.294) (width 0.25) (layer B.Cu) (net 4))
 (segment (start 48.7 47.132) (end 43.546 47.132) (width 0.25) (layer B.Cu) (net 4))
 (segment (start 43.434 47.244) (end 43.434 46.736) (width 0.25) (layer B.Cu) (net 4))
 (segment (start 43.546 47.132) (end 43.434 47.244) (width 0.25) (layer B.Cu) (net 4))
 (segment (start 43.434 65.786) (end 43.434 47.244) (width 0.25) (layer B.Cu) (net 4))
 (segment (start 112.21001 85.067402) (end 112.21001 76.29199) (width 0.25) (layer B.Cu) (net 6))
 (segment (start 91.920411 105.357001) (end 112.21001 85.067402) (width 0.25) (layer B.Cu) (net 6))
 (segment (start 112.21001 76.29199) (end 118.1 70.402) (width 0.25) (layer B.Cu) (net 6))
 (segment (start 68.493001 105.357001) (end 91.920411 105.357001) (width 0.25) (layer B.Cu) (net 6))
 (segment (start 68.072 104.936) (end 68.493001 105.357001) (width 0.25) (layer B.Cu) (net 6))
 (segment (start 68.072 104.936) (end 64.55 104.936) (width 0.25) (layer B.Cu) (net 6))
 (segment (start 68 47.132) (end 64.628 47.132) (width 0.25) (layer B.Cu) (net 6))
 (segment (start 64.628 47.132) (end 64.55 47.21) (width 0.25) (layer B.Cu) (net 6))
 (segment (start 64.55 47.21) (end 64.55 34.578) (width 0.25) (layer B.Cu) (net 6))
 (segment (start 64.618 66.074) (end 64.55 66.006) (width 0.25) (layer B.Cu) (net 6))
 (segment (start 68.072 66.074) (end 64.618 66.074) (width 0.25) (layer B.Cu) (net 6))
 (segment (start 64.55 66.006) (end 64.55 47.21) (width 0.25) (layer B.Cu) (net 6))
 (segment (start 64.804 85.632) (end 64.55 85.378) (width 0.25) (layer B.Cu) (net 6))
 (segment (start 68.072 85.632) (end 64.804 85.632) (width 0.25) (layer B.Cu) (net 6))
 (segment (start 64.55 85.378) (end 64.55 66.006) (width 0.25) (layer B.Cu) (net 6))
 (segment (start 64.55 104.936) (end 64.55 85.378) (width 0.25) (layer B.Cu) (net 6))
 (segment (start 68 39.472) (end 67.55 39.022) (width 0.25) (layer B.Cu) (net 5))
 (segment (start 68 45.032) (end 68 39.472) (width 0.25) (layer B.Cu) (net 5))
 (segment (start 87.3 39.572) (end 86.75 39.022) (width 0.25) (layer B.Cu) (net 7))
 (segment (start 87.3 45.232) (end 87.3 39.572) (width 0.25) (layer B.Cu) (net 7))
 (segment (start 91.909002 104.732) (end 111.76 84.881002) (width 0.25) (layer B.Cu) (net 8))
 (segment (start 86.8 104.732) (end 91.909002 104.732) (width 0.25) (layer B.Cu) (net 8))
 (segment (start 111.76 74.202) (end 118.1 67.862) (width 0.25) (layer B.Cu) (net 8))
 (segment (start 111.76 84.881002) (end 111.76 74.202) (width 0.25) (layer B.Cu) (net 8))
 (segment (start 86.8 104.732) (end 84.158 104.732) (width 0.25) (layer B.Cu) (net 8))
 (segment (start 84.158 104.732) (end 82.296 102.87) (width 0.25) (layer B.Cu) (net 8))
 (segment (start 82.296 102.87) (end 82.042 102.616) (width 0.25) (layer B.Cu) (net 8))
 (segment (start 82.076 85.378) (end 82.042 85.344) (width 0.25) (layer B.Cu) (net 8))
 (segment (start 87.63 85.378) (end 82.076 85.378) (width 0.25) (layer B.Cu) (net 8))
 (segment (start 82.042 102.616) (end 82.042 85.344) (width 0.25) (layer B.Cu) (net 8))
 (segment (start 87.376 66.328) (end 82.076 66.328) (width 0.25) (layer B.Cu) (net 8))
 (segment (start 82.076 66.328) (end 82.042 66.294) (width 0.25) (layer B.Cu) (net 8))
 (segment (start 82.042 85.344) (end 82.042 66.294) (width 0.25) (layer B.Cu) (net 8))
 (segment (start 82.208 47.332) (end 82.042 47.498) (width 0.25) (layer B.Cu) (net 8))
 (segment (start 87.3 47.332) (end 82.208 47.332) (width 0.25) (layer B.Cu) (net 8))
 (segment (start 82.042 47.958) (end 82.042 34.4825) (width 0.25) (layer B.Cu) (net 8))
 (segment (start 82.042 66.294) (end 82.042 47.958) (width 0.25) (layer B.Cu) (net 8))
 (segment (start 82.042 47.958) (end 82.042 47.498) (width 0.25) (layer B.Cu) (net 8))
 (segment (start 29.464 58.736) (end 29.05 58.322) (width 0.25) (layer B.Cu) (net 9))
 (segment (start 29.464 64.228) (end 29.464 58.736) (width 0.25) (layer B.Cu) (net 9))
 (segment (start 48.6 58.672) (end 48.25 58.322) (width 0.25) (layer B.Cu) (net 10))
 (segment (start 48.6 64.232) (end 48.6 58.672) (width 0.25) (layer B.Cu) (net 10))
 (segment (start 68.072 58.844) (end 67.55 58.322) (width 0.25) (layer B.Cu) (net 11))
 (segment (start 68.072 63.974) (end 68.072 58.844) (width 0.25) (layer B.Cu) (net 11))
 (segment (start 87.376 58.948) (end 86.75 58.322) (width 0.25) (layer B.Cu) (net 12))
 (segment (start 87.376 64.228) (end 87.376 58.948) (width 0.25) (layer B.Cu) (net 12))
 (segment (start 29.718 78.19) (end 29.05 77.522) (width 0.25) (layer B.Cu) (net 13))
 (segment (start 29.718 83.278) (end 29.718 78.19) (width 0.25) (layer B.Cu) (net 13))
 (segment (start 48.6 77.872) (end 48.25 77.522) (width 0.25) (layer B.Cu) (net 14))
 (segment (start 48.6 83.432) (end 48.6 77.872) (width 0.25) (layer B.Cu) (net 14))
 (segment (start 68.072 78.044) (end 67.55 77.522) (width 0.25) (layer B.Cu) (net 15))
 (segment (start 68.072 83.532) (end 68.072 78.044) (width 0.25) (layer B.Cu) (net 15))
 (segment (start 87.63 78.402) (end 86.75 77.522) (width 0.25) (layer B.Cu) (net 16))
 (segment (start 87.63 83.278) (end 87.63 78.402) (width 0.25) (layer B.Cu) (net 16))
 (segment (start 29.2 96.872) (end 29.05 96.722) (width 0.25) (layer B.Cu) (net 17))
 (segment (start 29.2 102.732) (end 29.2 96.872) (width 0.25) (layer B.Cu) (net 17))
 (segment (start 49.022 97.494) (end 48.25 96.722) (width 0.25) (layer B.Cu) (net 18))
 (segment (start 49.022 102.582) (end 49.022 97.494) (width 0.25) (layer B.Cu) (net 18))
 (segment (start 68.072 97.244) (end 67.55 96.722) (width 0.25) (layer B.Cu) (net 19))
 (segment (start 68.072 102.836) (end 68.072 97.244) (width 0.25) (layer B.Cu) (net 19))
 (segment (start 86.8 96.772) (end 86.75 96.722) (width 0.25) (layer B.Cu) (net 20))
 (segment (start 86.8 102.632) (end 86.8 96.772) (width 0.25) (layer B.Cu) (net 20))
 (segment (start 82.042 31.5575) (end 99.5755 31.5575) (width 0.5) (layer B.Cu) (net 21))
 (segment (start 64.7085 31.5575) (end 64.516 31.365) (width 0.5) (layer B.Cu) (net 21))
 (segment (start 82.042 31.5575) (end 64.7085 31.5575) (width 0.5) (layer B.Cu) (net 21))
 (segment (start 43.4955 31.365) (end 43.434 31.3035) (width 0.5) (layer B.Cu) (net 21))
 (segment (start 64.516 31.365) (end 43.4955 31.365) (width 0.5) (layer B.Cu) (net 21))
 (segment (start 43.434 31.3035) (end 24.384 31.3035) (width 0.5) (layer B.Cu) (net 21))
 (segment (start 99.5755 31.5575) (end 118.1 50.082) (width 0.5) (layer B.Cu) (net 21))
 (segment (start 93.1 85.242) (end 93.1 94.182) (width 0.25) (layer F.Cu) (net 25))
 (segment (start 93.1 94.182) (end 73.9 94.182) (width 0.25) (layer F.Cu) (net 25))
 (segment (start 73.9 94.182) (end 54.6 94.182) (width 0.25) (layer F.Cu) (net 25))
 (segment (start 54.6 94.182) (end 35.4 94.182) (width 0.25) (layer F.Cu) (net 25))
 (segment (start 118.1 60.242) (end 93.1 85.242) (width 0.25) (layer F.Cu) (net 25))
 (segment (start 110.38 57.702) (end 93.1 74.982) (width 0.25) (layer F.Cu) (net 24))
 (segment (start 93.1 74.982) (end 73.9 74.982) (width 0.25) (layer F.Cu) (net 24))
 (segment (start 73.9 74.982) (end 54.6 74.982) (width 0.25) (layer F.Cu) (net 24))
 (segment (start 54.6 74.982) (end 35.4 74.982) (width 0.25) (layer F.Cu) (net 24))
 (segment (start 118.1 57.702) (end 110.38 57.702) (width 0.25) (layer F.Cu) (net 24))
 (segment (start 93.72 55.162) (end 93.1 55.782) (width 0.25) (layer F.Cu) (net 23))
 (segment (start 93.1 55.782) (end 73.9 55.782) (width 0.25) (layer F.Cu) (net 23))
 (segment (start 73.9 55.782) (end 54.6 55.782) (width 0.25) (layer F.Cu) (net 23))
 (segment (start 54.6 55.782) (end 35.4 55.782) (width 0.25) (layer F.Cu) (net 23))
 (segment (start 118.1 55.162) (end 93.72 55.162) (width 0.25) (layer F.Cu) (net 23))
 (segment (start 109.24 52.622) (end 93.1 36.482) (width 0.25) (layer F.Cu) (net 22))
 (segment (start 93.1 36.482) (end 73.9 36.482) (width 0.25) (layer F.Cu) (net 22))
 (segment (start 73.9 36.482) (end 54.6 36.482) (width 0.25) (layer F.Cu) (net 22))
 (segment (start 54.6 36.482) (end 35.4 36.482) (width 0.25) (layer F.Cu) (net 22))
 (segment (start 118.1 52.622) (end 109.24 52.622) (width 0.25) (layer F.Cu) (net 22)))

